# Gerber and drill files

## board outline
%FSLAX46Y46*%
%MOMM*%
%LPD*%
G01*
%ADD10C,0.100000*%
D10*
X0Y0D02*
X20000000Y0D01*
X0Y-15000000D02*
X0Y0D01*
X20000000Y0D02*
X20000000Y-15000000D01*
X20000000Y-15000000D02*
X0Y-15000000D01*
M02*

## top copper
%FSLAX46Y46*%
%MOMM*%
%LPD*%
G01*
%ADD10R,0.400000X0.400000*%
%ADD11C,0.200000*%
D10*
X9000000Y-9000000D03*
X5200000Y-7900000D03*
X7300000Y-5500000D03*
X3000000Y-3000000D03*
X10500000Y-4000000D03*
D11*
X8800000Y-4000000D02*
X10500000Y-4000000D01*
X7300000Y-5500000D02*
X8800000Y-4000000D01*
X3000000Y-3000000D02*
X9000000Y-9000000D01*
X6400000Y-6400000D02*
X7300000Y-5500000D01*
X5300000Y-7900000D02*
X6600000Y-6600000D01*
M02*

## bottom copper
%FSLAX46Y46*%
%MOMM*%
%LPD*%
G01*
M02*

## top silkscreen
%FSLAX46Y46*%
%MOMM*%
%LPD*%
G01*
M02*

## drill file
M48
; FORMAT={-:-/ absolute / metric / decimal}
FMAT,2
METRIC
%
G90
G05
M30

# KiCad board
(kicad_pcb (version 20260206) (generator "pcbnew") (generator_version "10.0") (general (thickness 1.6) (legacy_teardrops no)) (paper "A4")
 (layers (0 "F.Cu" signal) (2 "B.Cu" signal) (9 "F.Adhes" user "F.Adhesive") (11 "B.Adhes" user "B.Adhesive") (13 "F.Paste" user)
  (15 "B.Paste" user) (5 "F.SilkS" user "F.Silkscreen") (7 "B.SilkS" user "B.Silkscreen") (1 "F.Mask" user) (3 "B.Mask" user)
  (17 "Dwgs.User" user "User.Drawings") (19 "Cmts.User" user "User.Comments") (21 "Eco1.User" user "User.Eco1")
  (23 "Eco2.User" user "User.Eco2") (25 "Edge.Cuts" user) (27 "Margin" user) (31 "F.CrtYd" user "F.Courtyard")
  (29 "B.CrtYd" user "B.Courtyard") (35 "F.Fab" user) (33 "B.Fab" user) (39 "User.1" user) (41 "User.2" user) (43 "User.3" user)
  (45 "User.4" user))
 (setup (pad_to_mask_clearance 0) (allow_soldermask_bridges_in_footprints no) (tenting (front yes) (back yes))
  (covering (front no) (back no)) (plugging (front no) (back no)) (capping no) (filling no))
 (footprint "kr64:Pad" (layer "F.Cu") (at 9 9)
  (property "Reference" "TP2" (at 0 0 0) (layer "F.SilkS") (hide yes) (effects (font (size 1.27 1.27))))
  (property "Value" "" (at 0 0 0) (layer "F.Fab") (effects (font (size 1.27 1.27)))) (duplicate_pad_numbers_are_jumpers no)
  (pad "1" smd rect (at 0 0) (size 0.4 0.4) (layers "F.Cu" "F.Mask" "F.Paste") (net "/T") (thermal_bridge_angle 45)))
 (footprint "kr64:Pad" (layer "F.Cu") (at 5.2 7.9)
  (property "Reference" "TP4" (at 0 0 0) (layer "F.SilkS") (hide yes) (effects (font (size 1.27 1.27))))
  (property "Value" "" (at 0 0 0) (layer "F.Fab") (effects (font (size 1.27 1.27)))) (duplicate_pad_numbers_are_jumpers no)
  (pad "1" smd rect (at 0 0) (size 0.4 0.4) (layers "F.Cu" "F.Mask" "F.Paste") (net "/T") (thermal_bridge_angle 45)))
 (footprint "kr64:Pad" (layer "F.Cu") (at 7.3 5.5)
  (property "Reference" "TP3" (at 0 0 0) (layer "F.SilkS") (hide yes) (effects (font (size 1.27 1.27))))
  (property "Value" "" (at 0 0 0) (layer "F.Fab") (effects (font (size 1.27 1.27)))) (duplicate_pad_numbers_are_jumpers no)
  (pad "1" smd rect (at 0 0) (size 0.4 0.4) (layers "F.Cu" "F.Mask" "F.Paste") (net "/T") (thermal_bridge_angle 45)))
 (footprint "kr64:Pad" (layer "F.Cu") (at 3 3)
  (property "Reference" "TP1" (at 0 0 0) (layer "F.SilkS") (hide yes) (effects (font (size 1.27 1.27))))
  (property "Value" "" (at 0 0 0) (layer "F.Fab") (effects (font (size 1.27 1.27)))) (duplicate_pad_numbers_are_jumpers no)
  (pad "1" smd rect (at 0 0) (size 0.4 0.4) (layers "F.Cu" "F.Mask" "F.Paste") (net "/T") (thermal_bridge_angle 45)))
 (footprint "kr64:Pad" (layer "F.Cu") (at 10.5 4)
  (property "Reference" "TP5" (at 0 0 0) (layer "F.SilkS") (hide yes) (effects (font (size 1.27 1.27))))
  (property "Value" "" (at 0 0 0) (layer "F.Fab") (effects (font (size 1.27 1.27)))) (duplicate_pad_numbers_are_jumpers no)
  (pad "1" smd rect (at 0 0) (size 0.4 0.4) (layers "F.Cu" "F.Mask" "F.Paste") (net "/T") (thermal_bridge_angle 45)))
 (gr_line (start 0 0) (end 20 0) (stroke (width 0.1) (type default)) (layer "Edge.Cuts"))
 (gr_line (start 0 15) (end 0 0) (stroke (width 0.1) (type default)) (layer "Edge.Cuts"))
 (gr_line (start 20 0) (end 20 15) (stroke (width 0.1) (type default)) (layer "Edge.Cuts"))
 (gr_line (start 20 15) (end 0 15) (stroke (width 0.1) (type default)) (layer "Edge.Cuts"))
 (segment (start 8.8 4) (end 10.5 4) (width 0.2) (layer "F.Cu") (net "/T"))
 (segment (start 7.3 5.5) (end 8.8 4) (width 0.2) (layer "F.Cu") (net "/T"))
 (segment (start 3 3) (end 9 9) (width 0.2) (layer "F.Cu") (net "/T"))
 (segment (start 6.4 6.4) (end 7.3 5.5) (width 0.2) (layer "F.Cu") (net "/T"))
 (segment (start 5.3 7.9) (end 6.6 6.6) (width 0.2) (layer "F.Cu") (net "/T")))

